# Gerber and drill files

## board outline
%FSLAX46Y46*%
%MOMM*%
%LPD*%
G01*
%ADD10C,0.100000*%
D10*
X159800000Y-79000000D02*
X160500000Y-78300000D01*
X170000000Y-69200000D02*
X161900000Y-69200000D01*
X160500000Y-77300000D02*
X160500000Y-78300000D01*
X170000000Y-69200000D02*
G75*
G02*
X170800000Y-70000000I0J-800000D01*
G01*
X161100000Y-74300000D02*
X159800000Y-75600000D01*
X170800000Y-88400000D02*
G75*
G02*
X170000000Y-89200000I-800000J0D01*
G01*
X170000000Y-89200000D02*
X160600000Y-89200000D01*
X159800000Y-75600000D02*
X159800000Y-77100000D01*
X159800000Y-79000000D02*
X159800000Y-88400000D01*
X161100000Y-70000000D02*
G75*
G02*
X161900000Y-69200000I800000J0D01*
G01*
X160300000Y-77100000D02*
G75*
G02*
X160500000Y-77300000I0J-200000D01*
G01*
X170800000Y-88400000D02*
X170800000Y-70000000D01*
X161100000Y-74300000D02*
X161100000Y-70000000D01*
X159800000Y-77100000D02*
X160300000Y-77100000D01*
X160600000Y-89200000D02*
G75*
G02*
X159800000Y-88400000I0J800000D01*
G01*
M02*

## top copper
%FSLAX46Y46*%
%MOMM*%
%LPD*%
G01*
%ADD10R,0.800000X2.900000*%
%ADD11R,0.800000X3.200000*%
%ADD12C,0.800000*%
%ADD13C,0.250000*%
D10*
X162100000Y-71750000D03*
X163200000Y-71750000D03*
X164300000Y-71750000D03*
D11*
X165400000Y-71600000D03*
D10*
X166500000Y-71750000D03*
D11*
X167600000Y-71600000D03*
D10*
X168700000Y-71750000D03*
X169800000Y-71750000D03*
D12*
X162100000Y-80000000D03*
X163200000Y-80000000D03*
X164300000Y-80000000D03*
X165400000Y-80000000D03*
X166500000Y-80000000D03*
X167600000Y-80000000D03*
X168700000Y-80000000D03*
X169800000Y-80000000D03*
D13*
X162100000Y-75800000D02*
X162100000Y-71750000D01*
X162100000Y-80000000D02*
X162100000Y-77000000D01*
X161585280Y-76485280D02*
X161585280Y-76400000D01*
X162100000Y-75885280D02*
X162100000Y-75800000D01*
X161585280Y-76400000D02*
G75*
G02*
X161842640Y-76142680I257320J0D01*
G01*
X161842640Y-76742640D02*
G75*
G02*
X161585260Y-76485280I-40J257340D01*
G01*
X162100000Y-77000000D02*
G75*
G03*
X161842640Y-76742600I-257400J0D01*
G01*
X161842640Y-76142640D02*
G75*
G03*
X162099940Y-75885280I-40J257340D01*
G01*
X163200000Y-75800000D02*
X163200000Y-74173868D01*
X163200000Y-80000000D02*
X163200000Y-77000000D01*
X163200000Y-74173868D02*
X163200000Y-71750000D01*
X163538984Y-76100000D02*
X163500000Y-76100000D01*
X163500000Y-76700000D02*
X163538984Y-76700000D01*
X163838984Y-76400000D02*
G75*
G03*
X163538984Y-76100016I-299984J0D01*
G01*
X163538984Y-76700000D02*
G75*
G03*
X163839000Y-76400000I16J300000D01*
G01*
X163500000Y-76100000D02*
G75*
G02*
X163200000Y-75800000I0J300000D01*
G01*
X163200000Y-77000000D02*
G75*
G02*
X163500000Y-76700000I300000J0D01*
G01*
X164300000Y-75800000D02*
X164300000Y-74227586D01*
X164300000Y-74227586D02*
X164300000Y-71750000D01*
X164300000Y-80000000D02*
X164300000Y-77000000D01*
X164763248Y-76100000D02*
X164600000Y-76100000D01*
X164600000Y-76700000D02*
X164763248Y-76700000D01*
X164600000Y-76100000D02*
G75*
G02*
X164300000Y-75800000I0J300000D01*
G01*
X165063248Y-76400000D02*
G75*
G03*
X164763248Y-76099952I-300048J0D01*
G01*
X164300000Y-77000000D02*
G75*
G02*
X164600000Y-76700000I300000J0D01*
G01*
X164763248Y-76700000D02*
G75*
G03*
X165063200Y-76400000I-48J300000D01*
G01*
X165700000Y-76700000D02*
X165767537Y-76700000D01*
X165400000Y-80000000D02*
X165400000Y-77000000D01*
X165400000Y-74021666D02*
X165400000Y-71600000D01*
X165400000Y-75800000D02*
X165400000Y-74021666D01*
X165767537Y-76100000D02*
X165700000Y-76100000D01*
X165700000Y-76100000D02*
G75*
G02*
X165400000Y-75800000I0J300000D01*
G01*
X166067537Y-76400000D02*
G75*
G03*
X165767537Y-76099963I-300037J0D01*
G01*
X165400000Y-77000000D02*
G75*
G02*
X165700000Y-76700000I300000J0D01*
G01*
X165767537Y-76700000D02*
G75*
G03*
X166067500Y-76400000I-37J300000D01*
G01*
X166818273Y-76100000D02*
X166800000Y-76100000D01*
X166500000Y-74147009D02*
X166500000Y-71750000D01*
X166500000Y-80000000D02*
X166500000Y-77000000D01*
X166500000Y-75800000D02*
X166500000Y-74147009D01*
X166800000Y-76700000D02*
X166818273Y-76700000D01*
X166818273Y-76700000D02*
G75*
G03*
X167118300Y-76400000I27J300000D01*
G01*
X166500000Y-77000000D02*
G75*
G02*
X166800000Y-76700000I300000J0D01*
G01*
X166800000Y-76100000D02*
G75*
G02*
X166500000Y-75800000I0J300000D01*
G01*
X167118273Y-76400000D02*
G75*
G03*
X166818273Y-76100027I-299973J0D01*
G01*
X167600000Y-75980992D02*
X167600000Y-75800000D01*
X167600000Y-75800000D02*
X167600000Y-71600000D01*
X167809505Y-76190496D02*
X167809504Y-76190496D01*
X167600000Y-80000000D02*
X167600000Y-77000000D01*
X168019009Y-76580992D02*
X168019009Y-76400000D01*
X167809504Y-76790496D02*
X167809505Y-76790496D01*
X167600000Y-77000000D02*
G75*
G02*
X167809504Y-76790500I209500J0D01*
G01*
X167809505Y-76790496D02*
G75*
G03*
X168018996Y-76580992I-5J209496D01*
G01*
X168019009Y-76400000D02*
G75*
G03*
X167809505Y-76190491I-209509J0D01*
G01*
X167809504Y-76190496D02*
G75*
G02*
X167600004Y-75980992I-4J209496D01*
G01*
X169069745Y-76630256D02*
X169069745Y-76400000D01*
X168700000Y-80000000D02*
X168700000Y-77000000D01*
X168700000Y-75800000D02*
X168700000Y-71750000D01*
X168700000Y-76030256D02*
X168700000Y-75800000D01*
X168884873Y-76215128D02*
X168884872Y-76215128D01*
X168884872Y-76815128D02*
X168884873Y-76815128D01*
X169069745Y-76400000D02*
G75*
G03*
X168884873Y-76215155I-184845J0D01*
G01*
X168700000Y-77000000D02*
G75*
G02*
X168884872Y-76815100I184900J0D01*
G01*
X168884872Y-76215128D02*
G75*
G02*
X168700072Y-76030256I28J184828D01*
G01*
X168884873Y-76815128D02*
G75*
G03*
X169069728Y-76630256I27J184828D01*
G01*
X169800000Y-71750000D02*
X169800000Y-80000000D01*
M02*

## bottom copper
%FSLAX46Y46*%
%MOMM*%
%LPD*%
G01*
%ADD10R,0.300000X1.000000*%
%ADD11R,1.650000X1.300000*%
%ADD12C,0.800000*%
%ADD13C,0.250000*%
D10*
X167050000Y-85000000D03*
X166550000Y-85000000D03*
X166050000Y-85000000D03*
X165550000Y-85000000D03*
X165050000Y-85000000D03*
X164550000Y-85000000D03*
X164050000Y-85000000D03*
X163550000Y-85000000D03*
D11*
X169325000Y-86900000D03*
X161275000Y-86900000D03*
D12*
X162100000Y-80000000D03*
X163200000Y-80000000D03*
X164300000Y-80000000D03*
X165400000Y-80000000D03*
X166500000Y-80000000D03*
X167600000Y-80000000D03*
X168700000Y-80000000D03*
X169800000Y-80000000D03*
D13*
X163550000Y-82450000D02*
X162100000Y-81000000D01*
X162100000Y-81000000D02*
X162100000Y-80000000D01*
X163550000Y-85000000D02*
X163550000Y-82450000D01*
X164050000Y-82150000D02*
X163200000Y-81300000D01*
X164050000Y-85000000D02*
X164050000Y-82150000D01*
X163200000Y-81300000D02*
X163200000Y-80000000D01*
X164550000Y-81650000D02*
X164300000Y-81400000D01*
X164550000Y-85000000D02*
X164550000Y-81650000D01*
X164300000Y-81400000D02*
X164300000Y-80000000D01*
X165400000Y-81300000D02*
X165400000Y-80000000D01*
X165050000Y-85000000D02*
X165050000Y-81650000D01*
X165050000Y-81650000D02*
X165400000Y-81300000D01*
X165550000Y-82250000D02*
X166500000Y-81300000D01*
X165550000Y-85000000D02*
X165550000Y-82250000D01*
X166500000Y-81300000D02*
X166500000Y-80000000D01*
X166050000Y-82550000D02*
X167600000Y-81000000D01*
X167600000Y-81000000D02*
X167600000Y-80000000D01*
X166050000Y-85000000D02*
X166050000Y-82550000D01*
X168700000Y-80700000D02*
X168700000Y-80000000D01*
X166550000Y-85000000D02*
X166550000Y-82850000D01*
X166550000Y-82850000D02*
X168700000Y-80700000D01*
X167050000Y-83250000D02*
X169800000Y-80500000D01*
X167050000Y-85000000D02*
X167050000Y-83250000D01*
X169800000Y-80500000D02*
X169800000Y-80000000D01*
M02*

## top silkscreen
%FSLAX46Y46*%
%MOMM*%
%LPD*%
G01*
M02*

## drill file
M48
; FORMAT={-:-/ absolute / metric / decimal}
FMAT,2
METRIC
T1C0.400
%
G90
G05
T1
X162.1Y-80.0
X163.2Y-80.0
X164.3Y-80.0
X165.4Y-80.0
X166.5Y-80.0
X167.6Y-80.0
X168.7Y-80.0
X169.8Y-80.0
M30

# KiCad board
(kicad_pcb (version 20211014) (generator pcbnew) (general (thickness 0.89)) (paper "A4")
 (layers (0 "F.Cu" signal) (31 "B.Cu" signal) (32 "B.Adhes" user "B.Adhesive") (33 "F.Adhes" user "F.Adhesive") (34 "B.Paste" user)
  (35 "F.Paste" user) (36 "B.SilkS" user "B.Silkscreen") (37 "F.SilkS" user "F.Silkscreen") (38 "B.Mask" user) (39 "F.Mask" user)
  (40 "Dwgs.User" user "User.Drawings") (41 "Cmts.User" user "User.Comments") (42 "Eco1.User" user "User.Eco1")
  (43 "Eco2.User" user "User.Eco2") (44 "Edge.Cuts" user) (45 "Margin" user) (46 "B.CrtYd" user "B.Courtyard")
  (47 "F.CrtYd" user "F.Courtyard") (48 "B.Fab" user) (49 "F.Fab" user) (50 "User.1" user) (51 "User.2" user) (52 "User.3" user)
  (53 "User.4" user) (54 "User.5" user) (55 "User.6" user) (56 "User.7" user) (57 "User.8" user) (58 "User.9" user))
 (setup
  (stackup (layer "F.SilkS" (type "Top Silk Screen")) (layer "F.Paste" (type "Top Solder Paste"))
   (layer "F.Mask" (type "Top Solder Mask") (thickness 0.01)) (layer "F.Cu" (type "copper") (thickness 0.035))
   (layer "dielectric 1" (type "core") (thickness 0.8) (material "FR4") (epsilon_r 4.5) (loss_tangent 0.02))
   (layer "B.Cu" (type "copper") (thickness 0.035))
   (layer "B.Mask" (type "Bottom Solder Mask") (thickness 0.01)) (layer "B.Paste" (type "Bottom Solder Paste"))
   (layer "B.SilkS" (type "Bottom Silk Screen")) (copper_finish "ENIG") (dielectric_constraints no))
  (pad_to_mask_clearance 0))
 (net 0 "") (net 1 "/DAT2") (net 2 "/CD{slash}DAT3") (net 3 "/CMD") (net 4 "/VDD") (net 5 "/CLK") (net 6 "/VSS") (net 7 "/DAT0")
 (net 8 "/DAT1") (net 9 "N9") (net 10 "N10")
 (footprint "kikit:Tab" (layer "F.Cu") (at 165.3 89.2 90)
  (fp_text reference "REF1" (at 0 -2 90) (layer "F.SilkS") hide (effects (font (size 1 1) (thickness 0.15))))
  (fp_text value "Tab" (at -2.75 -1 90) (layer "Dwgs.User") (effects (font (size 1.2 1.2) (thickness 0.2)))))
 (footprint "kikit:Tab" (layer "F.Cu") (at 170.8 73.9 180)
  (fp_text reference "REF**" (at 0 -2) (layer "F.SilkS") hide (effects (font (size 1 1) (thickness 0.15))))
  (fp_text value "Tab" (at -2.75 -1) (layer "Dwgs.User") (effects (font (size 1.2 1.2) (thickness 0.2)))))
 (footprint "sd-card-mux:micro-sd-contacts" (layer "F.Cu") (at 165.95 69.2)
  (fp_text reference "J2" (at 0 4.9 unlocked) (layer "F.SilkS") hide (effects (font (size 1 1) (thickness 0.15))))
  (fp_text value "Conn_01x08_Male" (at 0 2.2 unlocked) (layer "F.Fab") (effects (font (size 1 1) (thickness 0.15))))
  (pad "1" smd rect (at -3.85 2.55) (size 0.8 2.9) (layers "F.Cu" "F.Mask") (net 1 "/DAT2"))
  (pad "2" smd rect (at -2.75 2.55) (size 0.8 2.9) (layers "F.Cu" "F.Mask") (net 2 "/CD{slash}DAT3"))
  (pad "3" smd rect (at -1.65 2.55) (size 0.8 2.9) (layers "F.Cu" "F.Mask") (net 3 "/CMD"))
  (pad "4" smd rect (at -0.55 2.4) (size 0.8 3.2) (layers "F.Cu" "F.Mask") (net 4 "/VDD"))
  (pad "5" smd rect (at 0.55 2.55) (size 0.8 2.9) (layers "F.Cu" "F.Mask") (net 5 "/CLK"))
  (pad "6" smd rect (at 1.65 2.4) (size 0.8 3.2) (layers "F.Cu" "F.Mask") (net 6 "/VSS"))
  (pad "7" smd rect (at 2.75 2.55) (size 0.8 2.9) (layers "F.Cu" "F.Mask") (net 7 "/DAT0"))
  (pad "8" smd rect (at 3.85 2.55) (size 0.8 2.9) (layers "F.Cu" "F.Mask") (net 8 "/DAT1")))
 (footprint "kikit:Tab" (layer "F.Cu") (at 165.96 69.05 -90)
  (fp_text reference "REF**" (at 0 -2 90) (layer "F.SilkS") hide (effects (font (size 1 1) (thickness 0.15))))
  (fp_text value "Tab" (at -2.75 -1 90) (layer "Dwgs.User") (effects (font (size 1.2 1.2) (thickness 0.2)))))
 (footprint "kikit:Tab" (layer "F.Cu") (at 170.8 83 180)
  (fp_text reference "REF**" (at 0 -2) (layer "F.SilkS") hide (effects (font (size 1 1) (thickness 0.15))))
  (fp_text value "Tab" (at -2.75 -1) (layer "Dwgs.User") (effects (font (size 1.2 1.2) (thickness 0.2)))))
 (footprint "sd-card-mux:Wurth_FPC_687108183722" (layer "B.Cu") (at 165.3 85 180)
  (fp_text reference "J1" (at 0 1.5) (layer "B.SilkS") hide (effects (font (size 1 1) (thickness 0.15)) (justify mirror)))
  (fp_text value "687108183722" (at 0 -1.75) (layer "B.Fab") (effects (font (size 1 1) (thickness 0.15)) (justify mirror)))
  (pad "1" smd rect (at -1.75 0 180) (size 0.3 1) (layers "B.Cu" "B.Paste" "B.Mask") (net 8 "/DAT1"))
  (pad "2" smd rect (at -1.25 0 180) (size 0.3 1) (layers "B.Cu" "B.Paste" "B.Mask") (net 7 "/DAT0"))
  (pad "3" smd rect (at -0.75 0 180) (size 0.3 1) (layers "B.Cu" "B.Paste" "B.Mask") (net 6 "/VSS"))
  (pad "4" smd rect (at -0.25 0 180) (size 0.3 1) (layers "B.Cu" "B.Paste" "B.Mask") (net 5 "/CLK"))
  (pad "5" smd rect (at 0.25 0 180) (size 0.3 1) (layers "B.Cu" "B.Paste" "B.Mask") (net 4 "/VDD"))
  (pad "6" smd rect (at 0.75 0 180) (size 0.3 1) (layers "B.Cu" "B.Paste" "B.Mask") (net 3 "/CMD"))
  (pad "7" smd rect (at 1.25 0 180) (size 0.3 1) (layers "B.Cu" "B.Paste" "B.Mask") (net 2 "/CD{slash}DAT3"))
  (pad "8" smd rect (at 1.75 0 180) (size 0.3 1) (layers "B.Cu" "B.Paste" "B.Mask") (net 1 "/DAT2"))
  (pad "9" smd rect (at -4.025 -1.9 180) (size 1.65 1.3) (layers "B.Cu" "B.Paste" "B.Mask") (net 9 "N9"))
  (pad "10" smd rect (at 4.025 -1.9 180) (size 1.65 1.3) (layers "B.Cu" "B.Paste" "B.Mask") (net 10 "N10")))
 (gr_line (start 159.8 79) (end 160.5 78.3) (layer "Edge.Cuts") (width 0.1))
 (gr_line (start 170 69.2) (end 161.9 69.2) (layer "Edge.Cuts") (width 0.1))
 (gr_line (start 160.5 77.3) (end 160.5 78.3) (layer "Edge.Cuts") (width 0.1))
 (gr_arc (start 170 69.2) (mid 170.565685 69.434315) (end 170.8 70) (layer "Edge.Cuts") (width 0.1))
 (gr_line (start 161.1 74.3) (end 159.8 75.6) (layer "Edge.Cuts") (width 0.1))
 (gr_arc (start 170.8 88.4) (mid 170.565685 88.965685) (end 170 89.2) (layer "Edge.Cuts") (width 0.1))
 (gr_line (start 170 89.2) (end 160.6 89.2) (layer "Edge.Cuts") (width 0.1))
 (gr_line (start 159.8 75.6) (end 159.8 77.1) (layer "Edge.Cuts") (width 0.1))
 (gr_line (start 159.8 79) (end 159.8 88.4) (layer "Edge.Cuts") (width 0.1))
 (gr_arc (start 161.1 70) (mid 161.334315 69.434315) (end 161.9 69.2) (layer "Edge.Cuts") (width 0.1))
 (gr_arc (start 160.3 77.1) (mid 160.441421 77.158579) (end 160.5 77.3) (layer "Edge.Cuts") (width 0.1))
 (gr_line (start 170.8 88.4) (end 170.8 70) (layer "Edge.Cuts") (width 0.1))
 (gr_line (start 161.1 74.3) (end 161.1 70) (layer "Edge.Cuts") (width 0.1))
 (gr_line (start 159.8 77.1) (end 160.3 77.1) (layer "Edge.Cuts") (width 0.1))
 (gr_arc (start 160.6 89.2) (mid 160.034315 88.965685) (end 159.8 88.4) (layer "Edge.Cuts") (width 0.1))
 (segment (start 162.1 75.8) (end 162.1 71.75) (width 0.25) (layer "F.Cu") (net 1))
 (segment (start 162.1 80) (end 162.1 77) (width 0.25) (layer "F.Cu") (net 1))
 (segment (start 161.58528 76.48528) (end 161.58528 76.4) (width 0.25) (layer "F.Cu") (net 1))
 (segment (start 162.1 75.88528) (end 162.1 75.8) (width 0.25) (layer "F.Cu") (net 1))
 (via (at 162.1 80) (size 0.8) (drill 0.4) (layers "F.Cu" "B.Cu") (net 1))
 (arc (start 161.58528 76.4) (mid 161.660659 76.218019) (end 161.84264 76.14264) (width 0.25) (layer "F.Cu") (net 1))
 (arc (start 161.84264 76.74264) (mid 161.660659 76.667261) (end 161.58528 76.48528) (width 0.25) (layer "F.Cu") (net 1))
 (arc (start 162.1 77) (mid 162.024621 76.818019) (end 161.84264 76.74264) (width 0.25) (layer "F.Cu") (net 1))
 (arc (start 161.84264 76.14264) (mid 162.024621 76.067261) (end 162.1 75.88528) (width 0.25) (layer "F.Cu") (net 1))
 (segment (start 163.55 82.45) (end 162.1 81) (width 0.25) (layer "B.Cu") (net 1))
 (segment (start 162.1 81) (end 162.1 80) (width 0.25) (layer "B.Cu") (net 1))
 (segment (start 163.55 85) (end 163.55 82.45) (width 0.25) (layer "B.Cu") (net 1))
 (segment (start 163.2 75.8) (end 163.2 74.173868) (width 0.25) (layer "F.Cu") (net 2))
 (segment (start 163.2 80) (end 163.2 77) (width 0.25) (layer "F.Cu") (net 2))
 (segment (start 163.2 74.173868) (end 163.2 71.75) (width 0.25) (layer "F.Cu") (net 2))
 (segment (start 163.538984 76.1) (end 163.5 76.1) (width 0.25) (layer "F.Cu") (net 2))
 (segment (start 163.5 76.7) (end 163.538984 76.7) (width 0.25) (layer "F.Cu") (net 2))
 (via (at 163.2 80) (size 0.8) (drill 0.4) (layers "F.Cu" "B.Cu") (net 2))
 (arc (start 163.838984 76.4) (mid 163.751116 76.187868) (end 163.538984 76.1) (width 0.25) (layer "F.Cu") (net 2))
 (arc (start 163.538984 76.7) (mid 163.751116 76.612132) (end 163.838984 76.4) (width 0.25) (layer "F.Cu") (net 2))
 (arc (start 163.5 76.1) (mid 163.287868 76.012132) (end 163.2 75.8) (width 0.25) (layer "F.Cu") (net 2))
 (arc (start 163.2 77) (mid 163.287868 76.787868) (end 163.5 76.7) (width 0.25) (layer "F.Cu") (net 2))
 (segment (start 164.05 82.15) (end 163.2 81.3) (width 0.25) (layer "B.Cu") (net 2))
 (segment (start 164.05 85) (end 164.05 82.15) (width 0.25) (layer "B.Cu") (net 2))
 (segment (start 163.2 81.3) (end 163.2 80) (width 0.25) (layer "B.Cu") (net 2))
 (segment (start 164.3 75.8) (end 164.3 74.227586) (width 0.25) (layer "F.Cu") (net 3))
 (segment (start 164.3 74.227586) (end 164.3 71.75) (width 0.25) (layer "F.Cu") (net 3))
 (segment (start 164.3 80) (end 164.3 77) (width 0.25) (layer "F.Cu") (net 3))
 (segment (start 164.763248 76.1) (end 164.6 76.1) (width 0.25) (layer "F.Cu") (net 3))
 (segment (start 164.6 76.7) (end 164.763248 76.7) (width 0.25) (layer "F.Cu") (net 3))
 (via (at 164.3 80) (size 0.8) (drill 0.4) (layers "F.Cu" "B.Cu") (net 3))
 (arc (start 164.6 76.1) (mid 164.387868 76.012132) (end 164.3 75.8) (width 0.25) (layer "F.Cu") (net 3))
 (arc (start 165.063248 76.4) (mid 164.97538 76.187868) (end 164.763248 76.1) (width 0.25) (layer "F.Cu") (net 3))
 (arc (start 164.3 77) (mid 164.387868 76.787868) (end 164.6 76.7) (width 0.25) (layer "F.Cu") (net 3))
 (arc (start 164.763248 76.7) (mid 164.97538 76.612132) (end 165.063248 76.4) (width 0.25) (layer "F.Cu") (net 3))
 (segment (start 164.55 81.65) (end 164.3 81.4) (width 0.25) (layer "B.Cu") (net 3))
 (segment (start 164.55 85) (end 164.55 81.65) (width 0.25) (layer "B.Cu") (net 3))
 (segment (start 164.3 81.4) (end 164.3 80) (width 0.25) (layer "B.Cu") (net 3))
 (segment (start 165.7 76.7) (end 165.767537 76.7) (width 0.25) (layer "F.Cu") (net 4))
 (segment (start 165.4 80) (end 165.4 77) (width 0.25) (layer "F.Cu") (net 4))
 (segment (start 165.4 74.021666) (end 165.4 71.6) (width 0.25) (layer "F.Cu") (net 4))
 (segment (start 165.4 75.8) (end 165.4 74.021666) (width 0.25) (layer "F.Cu") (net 4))
 (segment (start 165.767537 76.1) (end 165.7 76.1) (width 0.25) (layer "F.Cu") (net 4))
 (via (at 165.4 80) (size 0.8) (drill 0.4) (layers "F.Cu" "B.Cu") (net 4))
 (arc (start 165.7 76.1) (mid 165.487868 76.012132) (end 165.4 75.8) (width 0.25) (layer "F.Cu") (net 4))
 (arc (start 166.067537 76.4) (mid 165.979669 76.187868) (end 165.767537 76.1) (width 0.25) (layer "F.Cu") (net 4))
 (arc (start 165.4 77) (mid 165.487868 76.787868) (end 165.7 76.7) (width 0.25) (layer "F.Cu") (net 4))
 (arc (start 165.767537 76.7) (mid 165.979669 76.612132) (end 166.067537 76.4) (width 0.25) (layer "F.Cu") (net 4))
 (segment (start 165.4 81.3) (end 165.4 80) (width 0.25) (layer "B.Cu") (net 4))
 (segment (start 165.05 85) (end 165.05 81.65) (width 0.25) (layer "B.Cu") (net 4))
 (segment (start 165.05 81.65) (end 165.4 81.3) (width 0.25) (layer "B.Cu") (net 4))
 (segment (start 166.818273 76.1) (end 166.8 76.1) (width 0.25) (layer "F.Cu") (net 5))
 (segment (start 166.5 74.147009) (end 166.5 71.75) (width 0.25) (layer "F.Cu") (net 5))
 (segment (start 166.5 80) (end 166.5 77) (width 0.25) (layer "F.Cu") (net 5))
 (segment (start 166.5 75.8) (end 166.5 74.147009) (width 0.25) (layer "F.Cu") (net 5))
 (segment (start 166.8 76.7) (end 166.818273 76.7) (width 0.25) (layer "F.Cu") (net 5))
 (via (at 166.5 80) (size 0.8) (drill 0.4) (layers "F.Cu" "B.Cu") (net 5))
 (arc (start 166.818273 76.7) (mid 167.030405 76.612132) (end 167.118273 76.4) (width 0.25) (layer "F.Cu") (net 5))
 (arc (start 166.5 77) (mid 166.587868 76.787868) (end 166.8 76.7) (width 0.25) (layer "F.Cu") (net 5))
 (arc (start 166.8 76.1) (mid 166.587868 76.012132) (end 166.5 75.8) (width 0.25) (layer "F.Cu") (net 5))
 (arc (start 167.118273 76.4) (mid 167.030405 76.187868) (end 166.818273 76.1) (width 0.25) (layer "F.Cu") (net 5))
 (segment (start 165.55 82.25) (end 166.5 81.3) (width 0.25) (layer "B.Cu") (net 5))
 (segment (start 165.55 85) (end 165.55 82.25) (width 0.25) (layer "B.Cu") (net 5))
 (segment (start 166.5 81.3) (end 166.5 80) (width 0.25) (layer "B.Cu") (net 5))
 (segment (start 167.6 75.980992) (end 167.6 75.8) (width 0.25) (layer "F.Cu") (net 6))
 (segment (start 167.6 75.8) (end 167.6 71.6) (width 0.25) (layer "F.Cu") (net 6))
 (segment (start 167.809505 76.190496) (end 167.809504 76.190496) (width 0.25) (layer "F.Cu") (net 6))
 (segment (start 167.6 80) (end 167.6 77) (width 0.25) (layer "F.Cu") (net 6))
 (segment (start 168.019009 76.580992) (end 168.019009 76.4) (width 0.25) (layer "F.Cu") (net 6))
 (segment (start 167.809504 76.790496) (end 167.809505 76.790496) (width 0.25) (layer "F.Cu") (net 6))
 (via (at 167.6 80) (size 0.8) (drill 0.4) (layers "F.Cu" "B.Cu") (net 6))
 (arc (start 167.6 77) (mid 167.661362 76.851858) (end 167.809504 76.790496) (width 0.25) (layer "F.Cu") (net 6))
 (arc (start 167.809505 76.790496) (mid 167.957647 76.729134) (end 168.019009 76.580992) (width 0.25) (layer "F.Cu") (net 6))
 (arc (start 168.019009 76.4) (mid 167.957647 76.251858) (end 167.809505 76.190496) (width 0.25) (layer "F.Cu") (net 6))
 (arc (start 167.809504 76.190496) (mid 167.661362 76.129134) (end 167.6 75.980992) (width 0.25) (layer "F.Cu") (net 6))
 (segment (start 166.05 82.55) (end 167.6 81) (width 0.25) (layer "B.Cu") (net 6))
 (segment (start 167.6 81) (end 167.6 80) (width 0.25) (layer "B.Cu") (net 6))
 (segment (start 166.05 85) (end 166.05 82.55) (width 0.25) (layer "B.Cu") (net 6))
 (segment (start 169.069745 76.630256) (end 169.069745 76.4) (width 0.25) (layer "F.Cu") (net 7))
 (segment (start 168.7 80) (end 168.7 77) (width 0.25) (layer "F.Cu") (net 7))
 (segment (start 168.7 75.8) (end 168.7 71.75) (width 0.25) (layer "F.Cu") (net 7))
 (segment (start 168.7 76.030256) (end 168.7 75.8) (width 0.25) (layer "F.Cu") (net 7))
 (segment (start 168.884873 76.215128) (end 168.884872 76.215128) (width 0.25) (layer "F.Cu") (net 7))
 (segment (start 168.884872 76.815128) (end 168.884873 76.815128) (width 0.25) (layer "F.Cu") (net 7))
 (via (at 168.7 80) (size 0.8) (drill 0.4) (layers "F.Cu" "B.Cu") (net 7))
 (arc (start 169.069745 76.4) (mid 169.015597 76.269276) (end 168.884873 76.215128) (width 0.25) (layer "F.Cu") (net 7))
 (arc (start 168.7 77) (mid 168.754148 76.869276) (end 168.884872 76.815128) (width 0.25) (layer "F.Cu") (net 7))
 (arc (start 168.884872 76.215128) (mid 168.754148 76.16098) (end 168.7 76.030256) (width 0.25) (layer "F.Cu") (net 7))
 (arc (start 168.884873 76.815128) (mid 169.015597 76.76098) (end 169.069745 76.630256) (width 0.25) (layer "F.Cu") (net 7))
 (segment (start 168.7 80.7) (end 168.7 80) (width 0.25) (layer "B.Cu") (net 7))
 (segment (start 166.55 85) (end 166.55 82.85) (width 0.25) (layer "B.Cu") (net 7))
 (segment (start 166.55 82.85) (end 168.7 80.7) (width 0.25) (layer "B.Cu") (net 7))
 (segment (start 169.8 71.75) (end 169.8 80) (width 0.25) (layer "F.Cu") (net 8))
 (via (at 169.8 80) (size 0.8) (drill 0.4) (layers "F.Cu" "B.Cu") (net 8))
 (segment (start 167.05 83.25) (end 169.8 80.5) (width 0.25) (layer "B.Cu") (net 8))
 (segment (start 167.05 85) (end 167.05 83.25) (width 0.25) (layer "B.Cu") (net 8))
 (segment (start 169.8 80.5) (end 169.8 80) (width 0.25) (layer "B.Cu") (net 8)))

